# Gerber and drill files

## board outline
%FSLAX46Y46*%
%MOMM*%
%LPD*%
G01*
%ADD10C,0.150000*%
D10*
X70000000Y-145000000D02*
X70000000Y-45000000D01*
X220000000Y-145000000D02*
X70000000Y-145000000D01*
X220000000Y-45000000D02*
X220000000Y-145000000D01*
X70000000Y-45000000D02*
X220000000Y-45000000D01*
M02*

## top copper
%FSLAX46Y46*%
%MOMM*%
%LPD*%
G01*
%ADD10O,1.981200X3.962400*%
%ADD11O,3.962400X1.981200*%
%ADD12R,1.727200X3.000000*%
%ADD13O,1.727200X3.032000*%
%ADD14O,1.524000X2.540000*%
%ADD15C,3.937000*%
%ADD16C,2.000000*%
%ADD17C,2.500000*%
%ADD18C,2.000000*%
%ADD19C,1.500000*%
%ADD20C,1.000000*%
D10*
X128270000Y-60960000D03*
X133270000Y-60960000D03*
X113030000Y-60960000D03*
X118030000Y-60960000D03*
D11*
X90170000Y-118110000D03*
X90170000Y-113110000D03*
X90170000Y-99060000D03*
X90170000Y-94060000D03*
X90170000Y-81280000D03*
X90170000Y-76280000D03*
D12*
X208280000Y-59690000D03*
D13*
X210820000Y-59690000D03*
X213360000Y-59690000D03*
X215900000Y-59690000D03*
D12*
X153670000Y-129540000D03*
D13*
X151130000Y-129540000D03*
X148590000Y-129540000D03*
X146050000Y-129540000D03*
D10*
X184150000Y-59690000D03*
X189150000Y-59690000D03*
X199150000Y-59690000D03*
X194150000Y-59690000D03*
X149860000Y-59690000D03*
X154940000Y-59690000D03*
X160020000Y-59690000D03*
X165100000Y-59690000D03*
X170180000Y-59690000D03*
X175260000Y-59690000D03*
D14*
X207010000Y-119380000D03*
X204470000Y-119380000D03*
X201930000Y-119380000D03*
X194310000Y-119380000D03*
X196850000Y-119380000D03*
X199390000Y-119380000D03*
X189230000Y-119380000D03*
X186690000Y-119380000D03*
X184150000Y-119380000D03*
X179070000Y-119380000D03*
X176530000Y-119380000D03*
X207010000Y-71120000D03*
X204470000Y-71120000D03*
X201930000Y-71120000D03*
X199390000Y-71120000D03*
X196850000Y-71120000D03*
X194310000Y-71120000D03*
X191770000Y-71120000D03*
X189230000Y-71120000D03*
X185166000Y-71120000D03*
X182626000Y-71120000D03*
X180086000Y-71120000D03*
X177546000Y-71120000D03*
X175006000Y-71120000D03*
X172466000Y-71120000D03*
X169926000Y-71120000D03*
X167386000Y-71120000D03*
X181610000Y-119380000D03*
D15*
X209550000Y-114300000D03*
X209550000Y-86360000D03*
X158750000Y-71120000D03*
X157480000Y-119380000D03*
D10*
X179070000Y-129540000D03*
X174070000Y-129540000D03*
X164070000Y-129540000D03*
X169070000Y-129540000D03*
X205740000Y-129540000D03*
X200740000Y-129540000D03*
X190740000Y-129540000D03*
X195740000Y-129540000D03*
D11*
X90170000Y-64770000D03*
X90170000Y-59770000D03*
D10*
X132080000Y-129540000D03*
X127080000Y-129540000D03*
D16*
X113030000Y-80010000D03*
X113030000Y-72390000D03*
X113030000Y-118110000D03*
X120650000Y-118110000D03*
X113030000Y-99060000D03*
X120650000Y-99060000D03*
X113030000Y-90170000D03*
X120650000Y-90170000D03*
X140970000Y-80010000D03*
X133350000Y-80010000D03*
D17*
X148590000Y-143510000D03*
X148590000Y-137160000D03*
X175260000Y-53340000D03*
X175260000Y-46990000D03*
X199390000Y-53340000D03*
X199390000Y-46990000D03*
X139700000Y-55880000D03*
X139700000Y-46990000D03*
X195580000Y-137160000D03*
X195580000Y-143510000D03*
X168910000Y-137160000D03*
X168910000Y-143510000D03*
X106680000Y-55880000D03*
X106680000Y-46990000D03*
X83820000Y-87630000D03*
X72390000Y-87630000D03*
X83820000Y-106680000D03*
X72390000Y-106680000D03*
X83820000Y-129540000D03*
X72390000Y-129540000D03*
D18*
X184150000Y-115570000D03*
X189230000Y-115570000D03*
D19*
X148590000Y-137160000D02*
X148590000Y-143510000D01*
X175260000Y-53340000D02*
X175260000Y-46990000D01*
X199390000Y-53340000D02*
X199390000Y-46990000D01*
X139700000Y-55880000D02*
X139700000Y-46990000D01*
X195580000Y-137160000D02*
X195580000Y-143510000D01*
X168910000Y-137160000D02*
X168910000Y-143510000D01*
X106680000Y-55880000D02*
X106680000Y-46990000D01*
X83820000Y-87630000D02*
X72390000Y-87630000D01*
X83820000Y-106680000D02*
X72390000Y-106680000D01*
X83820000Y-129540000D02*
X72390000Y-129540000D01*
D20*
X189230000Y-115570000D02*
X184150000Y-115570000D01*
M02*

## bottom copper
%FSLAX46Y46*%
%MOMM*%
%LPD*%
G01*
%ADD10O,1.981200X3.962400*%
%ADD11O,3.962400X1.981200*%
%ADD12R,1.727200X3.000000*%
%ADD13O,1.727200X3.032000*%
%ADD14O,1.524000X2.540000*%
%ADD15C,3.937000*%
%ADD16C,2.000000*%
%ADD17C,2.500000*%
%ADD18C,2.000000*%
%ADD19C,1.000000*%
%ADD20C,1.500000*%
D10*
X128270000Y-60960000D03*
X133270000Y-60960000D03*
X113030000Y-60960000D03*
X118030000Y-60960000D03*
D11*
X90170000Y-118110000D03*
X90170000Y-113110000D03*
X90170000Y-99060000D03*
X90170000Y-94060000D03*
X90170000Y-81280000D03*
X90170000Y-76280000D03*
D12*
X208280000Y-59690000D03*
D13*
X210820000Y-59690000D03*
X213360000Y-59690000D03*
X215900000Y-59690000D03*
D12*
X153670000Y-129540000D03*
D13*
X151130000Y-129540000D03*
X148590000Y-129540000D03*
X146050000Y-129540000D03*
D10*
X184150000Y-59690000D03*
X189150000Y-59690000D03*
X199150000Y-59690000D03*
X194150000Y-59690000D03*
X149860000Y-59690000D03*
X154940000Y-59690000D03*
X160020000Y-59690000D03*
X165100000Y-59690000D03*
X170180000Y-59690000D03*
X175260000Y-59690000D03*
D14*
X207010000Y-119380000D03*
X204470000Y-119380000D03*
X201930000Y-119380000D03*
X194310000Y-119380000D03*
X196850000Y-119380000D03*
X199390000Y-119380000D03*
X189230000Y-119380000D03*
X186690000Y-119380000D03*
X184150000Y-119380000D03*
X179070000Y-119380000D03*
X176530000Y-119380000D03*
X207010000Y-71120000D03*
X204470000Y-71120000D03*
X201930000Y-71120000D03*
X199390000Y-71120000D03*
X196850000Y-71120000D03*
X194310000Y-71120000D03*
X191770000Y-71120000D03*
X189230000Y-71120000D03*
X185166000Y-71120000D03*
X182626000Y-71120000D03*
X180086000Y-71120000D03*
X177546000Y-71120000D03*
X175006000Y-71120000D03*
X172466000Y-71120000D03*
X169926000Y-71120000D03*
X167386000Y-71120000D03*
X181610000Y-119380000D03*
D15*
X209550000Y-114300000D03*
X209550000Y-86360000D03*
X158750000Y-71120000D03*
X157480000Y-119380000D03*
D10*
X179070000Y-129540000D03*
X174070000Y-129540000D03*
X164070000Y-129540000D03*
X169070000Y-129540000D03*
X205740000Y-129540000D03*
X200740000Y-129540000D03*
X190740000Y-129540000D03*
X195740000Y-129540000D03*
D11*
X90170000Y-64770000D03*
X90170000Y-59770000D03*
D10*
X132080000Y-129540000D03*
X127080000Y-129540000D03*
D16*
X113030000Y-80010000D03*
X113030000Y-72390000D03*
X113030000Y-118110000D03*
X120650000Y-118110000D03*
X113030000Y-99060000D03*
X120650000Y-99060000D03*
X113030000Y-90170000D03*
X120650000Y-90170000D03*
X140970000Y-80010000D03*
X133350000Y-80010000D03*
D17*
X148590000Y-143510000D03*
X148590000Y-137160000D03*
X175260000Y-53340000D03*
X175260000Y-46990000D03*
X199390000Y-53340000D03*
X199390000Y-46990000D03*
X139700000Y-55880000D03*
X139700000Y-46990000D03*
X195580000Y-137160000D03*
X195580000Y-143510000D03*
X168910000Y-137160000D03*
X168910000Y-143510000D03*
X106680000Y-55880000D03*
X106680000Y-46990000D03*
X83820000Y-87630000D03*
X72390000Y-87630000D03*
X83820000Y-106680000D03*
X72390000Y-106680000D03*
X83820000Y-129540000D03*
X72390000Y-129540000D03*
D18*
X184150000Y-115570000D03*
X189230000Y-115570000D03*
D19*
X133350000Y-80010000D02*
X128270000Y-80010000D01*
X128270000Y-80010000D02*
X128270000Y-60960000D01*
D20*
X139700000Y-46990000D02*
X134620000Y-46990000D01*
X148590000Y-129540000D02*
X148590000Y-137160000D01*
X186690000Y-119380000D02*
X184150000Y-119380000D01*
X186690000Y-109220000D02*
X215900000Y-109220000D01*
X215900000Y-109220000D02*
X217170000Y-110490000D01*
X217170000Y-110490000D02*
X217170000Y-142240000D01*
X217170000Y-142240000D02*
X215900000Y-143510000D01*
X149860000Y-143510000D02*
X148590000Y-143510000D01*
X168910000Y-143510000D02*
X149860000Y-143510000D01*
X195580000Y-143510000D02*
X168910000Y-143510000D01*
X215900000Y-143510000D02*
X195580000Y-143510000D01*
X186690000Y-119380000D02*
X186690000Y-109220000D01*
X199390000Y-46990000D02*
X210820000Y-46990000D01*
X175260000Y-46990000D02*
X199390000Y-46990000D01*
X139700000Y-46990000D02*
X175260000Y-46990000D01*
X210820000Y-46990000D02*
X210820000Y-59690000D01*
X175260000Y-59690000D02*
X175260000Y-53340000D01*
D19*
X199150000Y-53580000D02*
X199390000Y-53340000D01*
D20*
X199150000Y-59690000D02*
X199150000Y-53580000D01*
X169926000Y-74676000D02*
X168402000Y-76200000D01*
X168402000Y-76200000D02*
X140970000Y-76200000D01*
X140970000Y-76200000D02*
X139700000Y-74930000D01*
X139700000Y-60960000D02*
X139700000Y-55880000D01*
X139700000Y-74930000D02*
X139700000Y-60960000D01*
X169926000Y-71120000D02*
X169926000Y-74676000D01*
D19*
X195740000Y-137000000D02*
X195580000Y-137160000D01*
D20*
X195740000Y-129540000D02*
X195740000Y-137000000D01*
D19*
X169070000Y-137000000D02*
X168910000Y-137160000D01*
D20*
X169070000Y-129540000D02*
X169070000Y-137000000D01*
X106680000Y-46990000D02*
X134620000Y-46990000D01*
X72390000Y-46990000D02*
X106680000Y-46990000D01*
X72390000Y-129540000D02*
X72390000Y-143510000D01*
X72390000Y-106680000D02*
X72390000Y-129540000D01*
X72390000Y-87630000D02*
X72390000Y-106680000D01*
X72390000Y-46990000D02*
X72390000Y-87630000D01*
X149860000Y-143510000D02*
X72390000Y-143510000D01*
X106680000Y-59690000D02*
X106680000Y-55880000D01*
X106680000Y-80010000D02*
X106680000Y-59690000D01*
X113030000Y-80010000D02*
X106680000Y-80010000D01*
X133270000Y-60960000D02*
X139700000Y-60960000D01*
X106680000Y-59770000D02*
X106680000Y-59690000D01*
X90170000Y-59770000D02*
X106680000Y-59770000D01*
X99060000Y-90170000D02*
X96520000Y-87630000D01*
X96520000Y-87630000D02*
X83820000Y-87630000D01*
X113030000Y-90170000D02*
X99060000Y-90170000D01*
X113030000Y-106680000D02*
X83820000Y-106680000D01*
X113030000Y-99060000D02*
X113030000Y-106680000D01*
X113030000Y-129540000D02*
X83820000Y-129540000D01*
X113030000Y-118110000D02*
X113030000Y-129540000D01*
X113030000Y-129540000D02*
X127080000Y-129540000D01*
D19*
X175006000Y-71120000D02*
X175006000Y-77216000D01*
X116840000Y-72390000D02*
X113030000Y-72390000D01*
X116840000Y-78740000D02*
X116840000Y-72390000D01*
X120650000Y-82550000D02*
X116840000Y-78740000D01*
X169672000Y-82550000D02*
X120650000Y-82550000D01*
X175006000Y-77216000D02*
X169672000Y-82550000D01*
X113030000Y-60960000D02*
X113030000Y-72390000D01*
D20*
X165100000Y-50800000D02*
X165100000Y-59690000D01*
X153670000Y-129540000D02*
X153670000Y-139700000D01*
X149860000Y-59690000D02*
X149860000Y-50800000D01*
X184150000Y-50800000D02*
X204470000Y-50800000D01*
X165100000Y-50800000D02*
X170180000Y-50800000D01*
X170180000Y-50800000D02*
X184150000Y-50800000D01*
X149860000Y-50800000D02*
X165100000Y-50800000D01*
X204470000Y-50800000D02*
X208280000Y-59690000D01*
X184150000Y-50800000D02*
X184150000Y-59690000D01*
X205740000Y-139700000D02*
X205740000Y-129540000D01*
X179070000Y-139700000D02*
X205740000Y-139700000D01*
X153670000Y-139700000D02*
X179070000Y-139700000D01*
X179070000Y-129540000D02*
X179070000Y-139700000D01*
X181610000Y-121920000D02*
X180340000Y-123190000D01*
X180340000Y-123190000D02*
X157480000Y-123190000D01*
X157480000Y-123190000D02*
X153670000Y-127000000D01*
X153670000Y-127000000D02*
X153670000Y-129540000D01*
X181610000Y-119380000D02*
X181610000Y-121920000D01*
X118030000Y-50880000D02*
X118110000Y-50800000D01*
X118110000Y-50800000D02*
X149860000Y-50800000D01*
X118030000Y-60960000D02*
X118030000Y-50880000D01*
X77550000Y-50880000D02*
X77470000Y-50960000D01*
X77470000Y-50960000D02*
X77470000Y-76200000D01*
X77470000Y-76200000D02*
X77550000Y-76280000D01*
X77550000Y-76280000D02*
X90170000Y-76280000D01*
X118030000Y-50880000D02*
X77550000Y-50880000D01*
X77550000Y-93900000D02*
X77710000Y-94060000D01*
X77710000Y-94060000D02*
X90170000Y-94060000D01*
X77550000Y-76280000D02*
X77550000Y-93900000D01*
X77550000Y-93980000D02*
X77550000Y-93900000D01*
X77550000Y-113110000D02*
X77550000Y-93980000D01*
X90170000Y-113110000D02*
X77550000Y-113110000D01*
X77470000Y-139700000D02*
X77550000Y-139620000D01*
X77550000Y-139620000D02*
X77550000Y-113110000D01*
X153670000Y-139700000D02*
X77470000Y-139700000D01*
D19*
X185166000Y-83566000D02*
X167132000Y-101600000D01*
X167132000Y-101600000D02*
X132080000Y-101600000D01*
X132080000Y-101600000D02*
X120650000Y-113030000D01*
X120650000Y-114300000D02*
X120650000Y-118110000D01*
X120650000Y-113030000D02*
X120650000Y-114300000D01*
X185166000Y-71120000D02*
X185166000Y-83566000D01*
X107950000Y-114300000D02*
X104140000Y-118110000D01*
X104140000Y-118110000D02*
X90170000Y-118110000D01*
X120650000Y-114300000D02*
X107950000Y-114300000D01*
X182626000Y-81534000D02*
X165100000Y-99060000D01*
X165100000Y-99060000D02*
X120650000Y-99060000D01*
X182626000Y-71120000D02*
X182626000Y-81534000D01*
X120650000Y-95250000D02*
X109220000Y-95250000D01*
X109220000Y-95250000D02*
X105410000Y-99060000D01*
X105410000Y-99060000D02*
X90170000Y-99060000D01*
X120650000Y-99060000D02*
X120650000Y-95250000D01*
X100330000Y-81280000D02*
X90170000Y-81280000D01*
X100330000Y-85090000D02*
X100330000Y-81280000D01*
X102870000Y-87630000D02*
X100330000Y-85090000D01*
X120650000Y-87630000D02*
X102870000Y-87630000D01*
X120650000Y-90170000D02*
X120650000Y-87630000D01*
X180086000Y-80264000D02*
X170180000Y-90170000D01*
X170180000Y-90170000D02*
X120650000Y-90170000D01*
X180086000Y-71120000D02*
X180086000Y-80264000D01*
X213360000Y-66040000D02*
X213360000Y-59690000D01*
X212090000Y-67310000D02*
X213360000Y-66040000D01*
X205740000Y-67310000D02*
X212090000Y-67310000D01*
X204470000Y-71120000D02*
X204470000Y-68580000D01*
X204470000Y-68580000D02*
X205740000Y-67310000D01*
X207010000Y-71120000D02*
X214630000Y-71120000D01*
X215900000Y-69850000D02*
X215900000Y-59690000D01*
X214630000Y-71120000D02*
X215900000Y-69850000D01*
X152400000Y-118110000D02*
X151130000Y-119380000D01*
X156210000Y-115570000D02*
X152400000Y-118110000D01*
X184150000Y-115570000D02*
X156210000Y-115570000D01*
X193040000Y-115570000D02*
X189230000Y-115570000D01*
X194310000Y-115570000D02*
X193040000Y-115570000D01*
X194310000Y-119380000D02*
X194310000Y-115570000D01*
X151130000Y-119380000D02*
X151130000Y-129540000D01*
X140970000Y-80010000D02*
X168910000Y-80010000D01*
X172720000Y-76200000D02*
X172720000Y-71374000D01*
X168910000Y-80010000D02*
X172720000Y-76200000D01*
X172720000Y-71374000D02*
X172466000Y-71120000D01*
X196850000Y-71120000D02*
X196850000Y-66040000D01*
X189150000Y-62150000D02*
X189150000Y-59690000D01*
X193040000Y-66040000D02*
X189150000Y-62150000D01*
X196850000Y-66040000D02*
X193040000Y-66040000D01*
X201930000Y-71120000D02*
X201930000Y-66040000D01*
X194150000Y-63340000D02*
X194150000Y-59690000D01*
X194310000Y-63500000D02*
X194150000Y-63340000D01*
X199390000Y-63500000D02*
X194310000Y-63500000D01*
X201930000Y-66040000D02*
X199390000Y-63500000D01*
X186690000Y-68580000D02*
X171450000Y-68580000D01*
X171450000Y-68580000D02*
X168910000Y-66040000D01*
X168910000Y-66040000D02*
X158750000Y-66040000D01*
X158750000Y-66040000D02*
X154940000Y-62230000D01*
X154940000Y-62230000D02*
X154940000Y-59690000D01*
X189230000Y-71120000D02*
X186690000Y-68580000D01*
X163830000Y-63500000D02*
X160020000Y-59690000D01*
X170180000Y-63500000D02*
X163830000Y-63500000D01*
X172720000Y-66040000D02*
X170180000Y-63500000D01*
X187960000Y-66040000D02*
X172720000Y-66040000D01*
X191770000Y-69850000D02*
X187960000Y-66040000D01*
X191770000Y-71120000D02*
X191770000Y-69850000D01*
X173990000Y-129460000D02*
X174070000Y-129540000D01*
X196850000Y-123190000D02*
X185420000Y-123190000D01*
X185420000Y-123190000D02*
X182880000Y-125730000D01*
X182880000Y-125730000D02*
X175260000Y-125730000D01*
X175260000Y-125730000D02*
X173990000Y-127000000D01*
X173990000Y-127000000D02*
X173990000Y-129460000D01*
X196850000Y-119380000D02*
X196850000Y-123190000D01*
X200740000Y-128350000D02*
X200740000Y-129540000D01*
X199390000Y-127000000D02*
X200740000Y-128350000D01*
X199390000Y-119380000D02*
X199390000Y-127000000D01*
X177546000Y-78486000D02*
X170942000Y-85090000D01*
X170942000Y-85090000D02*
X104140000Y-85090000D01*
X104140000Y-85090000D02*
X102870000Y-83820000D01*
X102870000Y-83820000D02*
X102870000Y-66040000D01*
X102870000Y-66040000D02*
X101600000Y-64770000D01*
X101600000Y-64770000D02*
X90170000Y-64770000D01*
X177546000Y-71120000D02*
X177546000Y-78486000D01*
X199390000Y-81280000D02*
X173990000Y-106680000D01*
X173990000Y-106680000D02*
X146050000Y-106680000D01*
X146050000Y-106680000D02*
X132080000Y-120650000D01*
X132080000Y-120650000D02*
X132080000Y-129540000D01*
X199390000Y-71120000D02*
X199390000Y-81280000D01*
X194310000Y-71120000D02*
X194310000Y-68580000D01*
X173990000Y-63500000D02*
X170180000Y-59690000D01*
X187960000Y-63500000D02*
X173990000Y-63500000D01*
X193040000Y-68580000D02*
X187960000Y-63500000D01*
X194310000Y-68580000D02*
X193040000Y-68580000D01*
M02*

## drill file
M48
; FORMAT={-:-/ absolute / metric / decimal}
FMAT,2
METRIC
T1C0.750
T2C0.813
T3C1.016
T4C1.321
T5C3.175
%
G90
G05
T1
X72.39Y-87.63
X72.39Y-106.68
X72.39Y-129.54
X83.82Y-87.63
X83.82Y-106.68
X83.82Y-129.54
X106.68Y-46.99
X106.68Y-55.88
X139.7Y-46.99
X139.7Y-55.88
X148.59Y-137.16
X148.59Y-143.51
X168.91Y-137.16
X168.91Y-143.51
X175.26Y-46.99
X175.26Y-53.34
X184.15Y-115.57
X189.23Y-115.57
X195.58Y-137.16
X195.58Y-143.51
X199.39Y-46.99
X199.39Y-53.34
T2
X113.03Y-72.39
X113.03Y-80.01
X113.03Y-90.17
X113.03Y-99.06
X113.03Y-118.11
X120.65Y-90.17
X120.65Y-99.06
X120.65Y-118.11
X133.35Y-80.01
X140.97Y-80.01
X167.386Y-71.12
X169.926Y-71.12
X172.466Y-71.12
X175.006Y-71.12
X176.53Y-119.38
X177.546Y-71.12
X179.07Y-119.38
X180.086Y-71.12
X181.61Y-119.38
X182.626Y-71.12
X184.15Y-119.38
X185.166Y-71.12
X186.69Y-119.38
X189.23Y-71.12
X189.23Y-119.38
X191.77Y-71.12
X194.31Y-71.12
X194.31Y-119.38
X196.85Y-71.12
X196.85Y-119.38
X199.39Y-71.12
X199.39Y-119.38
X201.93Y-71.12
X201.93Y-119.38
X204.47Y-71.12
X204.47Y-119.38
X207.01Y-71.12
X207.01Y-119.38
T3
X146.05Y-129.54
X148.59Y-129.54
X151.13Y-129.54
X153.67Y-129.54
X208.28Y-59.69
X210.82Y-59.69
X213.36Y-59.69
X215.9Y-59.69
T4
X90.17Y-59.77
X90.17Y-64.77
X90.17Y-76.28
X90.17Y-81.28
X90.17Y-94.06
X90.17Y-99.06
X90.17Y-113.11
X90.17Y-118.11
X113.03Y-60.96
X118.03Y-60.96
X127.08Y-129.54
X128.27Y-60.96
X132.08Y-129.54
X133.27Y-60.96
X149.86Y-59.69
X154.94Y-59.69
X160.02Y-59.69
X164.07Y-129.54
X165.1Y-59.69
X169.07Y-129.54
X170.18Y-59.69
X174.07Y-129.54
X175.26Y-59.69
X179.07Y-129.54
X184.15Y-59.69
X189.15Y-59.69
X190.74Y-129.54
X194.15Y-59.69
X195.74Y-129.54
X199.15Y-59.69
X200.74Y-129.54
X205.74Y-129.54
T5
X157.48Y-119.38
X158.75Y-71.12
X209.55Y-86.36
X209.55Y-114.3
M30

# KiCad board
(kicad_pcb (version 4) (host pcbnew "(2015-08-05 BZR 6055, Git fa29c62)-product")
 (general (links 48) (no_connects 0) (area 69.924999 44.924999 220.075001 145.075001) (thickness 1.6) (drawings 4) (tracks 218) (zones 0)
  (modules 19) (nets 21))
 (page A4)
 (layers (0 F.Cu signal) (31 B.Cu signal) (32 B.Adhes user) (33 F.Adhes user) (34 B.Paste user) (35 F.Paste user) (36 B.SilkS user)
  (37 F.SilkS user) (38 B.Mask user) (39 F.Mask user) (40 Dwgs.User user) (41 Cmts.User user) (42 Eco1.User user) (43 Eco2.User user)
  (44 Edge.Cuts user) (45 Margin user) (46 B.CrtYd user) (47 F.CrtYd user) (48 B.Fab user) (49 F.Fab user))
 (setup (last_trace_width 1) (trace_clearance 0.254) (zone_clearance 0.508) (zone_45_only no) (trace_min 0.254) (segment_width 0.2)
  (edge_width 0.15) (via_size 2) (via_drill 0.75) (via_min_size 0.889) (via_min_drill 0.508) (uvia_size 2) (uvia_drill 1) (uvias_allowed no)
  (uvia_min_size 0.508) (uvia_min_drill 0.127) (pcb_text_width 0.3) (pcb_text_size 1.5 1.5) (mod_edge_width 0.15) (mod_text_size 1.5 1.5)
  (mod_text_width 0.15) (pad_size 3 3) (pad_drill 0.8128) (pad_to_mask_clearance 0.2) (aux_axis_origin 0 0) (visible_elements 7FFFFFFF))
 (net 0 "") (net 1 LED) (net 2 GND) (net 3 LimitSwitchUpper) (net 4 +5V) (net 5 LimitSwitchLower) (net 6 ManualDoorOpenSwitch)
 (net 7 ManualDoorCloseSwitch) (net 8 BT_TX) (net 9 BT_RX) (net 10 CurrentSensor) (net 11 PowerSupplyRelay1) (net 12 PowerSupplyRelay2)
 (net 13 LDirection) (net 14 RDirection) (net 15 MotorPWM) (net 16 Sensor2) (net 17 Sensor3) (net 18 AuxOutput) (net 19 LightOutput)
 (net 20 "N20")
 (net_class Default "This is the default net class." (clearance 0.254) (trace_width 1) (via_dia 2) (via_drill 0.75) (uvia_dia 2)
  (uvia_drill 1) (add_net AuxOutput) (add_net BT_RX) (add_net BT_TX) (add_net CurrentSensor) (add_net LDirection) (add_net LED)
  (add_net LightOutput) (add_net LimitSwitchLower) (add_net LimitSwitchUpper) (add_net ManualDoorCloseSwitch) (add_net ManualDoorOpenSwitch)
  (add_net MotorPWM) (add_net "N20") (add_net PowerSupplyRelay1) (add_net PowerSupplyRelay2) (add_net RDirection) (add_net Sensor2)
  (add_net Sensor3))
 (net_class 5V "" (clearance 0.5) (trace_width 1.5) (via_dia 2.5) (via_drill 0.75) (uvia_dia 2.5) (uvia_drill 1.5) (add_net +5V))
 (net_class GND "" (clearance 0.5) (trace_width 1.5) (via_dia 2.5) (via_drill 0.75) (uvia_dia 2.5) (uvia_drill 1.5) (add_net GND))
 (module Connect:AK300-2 (layer F.Cu) (at 128.27 60.96)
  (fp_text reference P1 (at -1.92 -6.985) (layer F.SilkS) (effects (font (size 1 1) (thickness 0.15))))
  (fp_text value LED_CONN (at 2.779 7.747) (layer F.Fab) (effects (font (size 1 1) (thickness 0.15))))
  (pad 1 thru_hole oval (at 0 0) (size 1.9812 3.9624) (drill 1.3208) (layers *.Cu F.Paste F.SilkS F.Mask) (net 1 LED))
  (pad 2 thru_hole oval (at 5 0) (size 1.9812 3.9624) (drill 1.3208) (layers *.Cu F.Paste F.SilkS F.Mask) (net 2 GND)))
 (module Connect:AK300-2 (layer F.Cu) (at 113.03 60.96)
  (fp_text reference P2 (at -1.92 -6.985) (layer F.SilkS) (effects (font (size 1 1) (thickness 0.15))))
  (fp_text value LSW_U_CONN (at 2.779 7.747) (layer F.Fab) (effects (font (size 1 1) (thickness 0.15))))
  (pad 1 thru_hole oval (at 0 0) (size 1.9812 3.9624) (drill 1.3208) (layers *.Cu F.Paste F.SilkS F.Mask) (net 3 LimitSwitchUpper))
  (pad 2 thru_hole oval (at 5 0) (size 1.9812 3.9624) (drill 1.3208) (layers *.Cu F.Paste F.SilkS F.Mask) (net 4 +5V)))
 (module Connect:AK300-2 (layer F.Cu) (at 90.17 118.11 90)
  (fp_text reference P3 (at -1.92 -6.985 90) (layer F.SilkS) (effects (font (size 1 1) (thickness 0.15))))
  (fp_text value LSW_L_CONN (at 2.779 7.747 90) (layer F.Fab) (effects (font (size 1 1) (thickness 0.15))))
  (pad 1 thru_hole oval (at 0 0 90) (size 1.9812 3.9624) (drill 1.3208) (layers *.Cu F.Paste F.SilkS F.Mask) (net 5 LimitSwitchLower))
  (pad 2 thru_hole oval (at 5 0 90) (size 1.9812 3.9624) (drill 1.3208) (layers *.Cu F.Paste F.SilkS F.Mask) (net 4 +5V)))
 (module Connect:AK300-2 (layer F.Cu) (at 90.17 99.06 90)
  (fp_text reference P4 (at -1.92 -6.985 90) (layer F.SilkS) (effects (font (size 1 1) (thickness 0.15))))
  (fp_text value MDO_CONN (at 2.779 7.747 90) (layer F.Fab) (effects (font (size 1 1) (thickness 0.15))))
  (pad 1 thru_hole oval (at 0 0 90) (size 1.9812 3.9624) (drill 1.3208) (layers *.Cu F.Paste F.SilkS F.Mask) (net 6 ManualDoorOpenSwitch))
  (pad 2 thru_hole oval (at 5 0 90) (size 1.9812 3.9624) (drill 1.3208) (layers *.Cu F.Paste F.SilkS F.Mask) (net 4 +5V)))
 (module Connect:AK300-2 (layer F.Cu) (at 90.17 81.28 90)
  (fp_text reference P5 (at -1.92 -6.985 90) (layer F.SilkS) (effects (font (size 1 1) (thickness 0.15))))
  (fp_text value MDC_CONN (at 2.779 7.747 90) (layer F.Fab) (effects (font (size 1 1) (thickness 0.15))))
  (pad 1 thru_hole oval (at 0 0 90) (size 1.9812 3.9624) (drill 1.3208) (layers *.Cu F.Paste F.SilkS F.Mask) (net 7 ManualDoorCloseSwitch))
  (pad 2 thru_hole oval (at 5 0 90) (size 1.9812 3.9624) (drill 1.3208) (layers *.Cu F.Paste F.SilkS F.Mask) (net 4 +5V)))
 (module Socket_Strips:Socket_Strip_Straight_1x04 (layer F.Cu) (at 208.28 59.69)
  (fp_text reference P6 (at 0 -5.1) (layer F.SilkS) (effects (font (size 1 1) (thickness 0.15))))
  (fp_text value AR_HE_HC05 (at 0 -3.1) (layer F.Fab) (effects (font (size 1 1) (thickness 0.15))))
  (pad 1 thru_hole rect (at 0 0) (size 1.7272 3) (drill 1.016) (layers *.Cu *.Mask F.SilkS) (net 4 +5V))
  (pad 2 thru_hole oval (at 2.54 0) (size 1.7272 3.032) (drill 1.016) (layers *.Cu *.Mask F.SilkS) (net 2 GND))
  (pad 3 thru_hole oval (at 5.08 0) (size 1.7272 3.032) (drill 1.016) (layers *.Cu *.Mask F.SilkS) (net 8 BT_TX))
  (pad 4 thru_hole oval (at 7.62 0) (size 1.7272 3.032) (drill 1.016) (layers *.Cu *.Mask F.SilkS) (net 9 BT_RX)))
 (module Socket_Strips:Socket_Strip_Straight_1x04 (layer F.Cu) (at 153.67 129.54 180)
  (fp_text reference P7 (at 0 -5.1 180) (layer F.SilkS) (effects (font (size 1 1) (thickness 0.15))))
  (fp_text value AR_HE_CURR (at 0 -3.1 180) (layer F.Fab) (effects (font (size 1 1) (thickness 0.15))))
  (pad 1 thru_hole rect (at 0 0 180) (size 1.7272 3) (drill 1.016) (layers *.Cu *.Mask F.SilkS) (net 4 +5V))
  (pad 2 thru_hole oval (at 2.54 0 180) (size 1.7272 3.032) (drill 1.016) (layers *.Cu *.Mask F.SilkS) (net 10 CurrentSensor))
  (pad 3 thru_hole oval (at 5.08 0 180) (size 1.7272 3.032) (drill 1.016) (layers *.Cu *.Mask F.SilkS) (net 2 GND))
  (pad 4 thru_hole oval (at 7.62 0 180) (size 1.7272 3.032) (drill 1.016) (layers *.Cu *.Mask F.SilkS)))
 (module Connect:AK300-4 (layer F.Cu) (at 184.15 59.69)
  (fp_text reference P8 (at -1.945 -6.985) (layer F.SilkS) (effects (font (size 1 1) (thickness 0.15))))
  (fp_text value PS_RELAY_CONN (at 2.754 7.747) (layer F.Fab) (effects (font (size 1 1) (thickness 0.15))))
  (pad 1 thru_hole oval (at 0 0) (size 1.9812 3.9624) (drill 1.3208) (layers *.Cu F.Paste F.SilkS F.Mask) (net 4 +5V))
  (pad 2 thru_hole oval (at 5 0) (size 1.9812 3.9624) (drill 1.3208) (layers *.Cu F.Paste F.SilkS F.Mask) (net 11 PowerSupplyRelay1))
  (pad 4 thru_hole oval (at 15 0) (size 1.9812 3.9624) (drill 1.3208) (layers *.Cu F.Paste F.SilkS F.Mask) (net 2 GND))
  (pad 3 thru_hole oval (at 10 0) (size 1.9812 3.9624) (drill 1.3208) (layers *.Cu *.Mask F.SilkS) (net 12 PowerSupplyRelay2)))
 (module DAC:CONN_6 (layer F.Cu) (at 162.56 59.69)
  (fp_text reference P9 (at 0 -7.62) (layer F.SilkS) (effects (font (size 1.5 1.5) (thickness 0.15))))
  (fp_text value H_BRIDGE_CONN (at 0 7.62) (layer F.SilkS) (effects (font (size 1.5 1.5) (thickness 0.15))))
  (pad 1 thru_hole oval (at -12.7 0) (size 1.9812 3.9624) (drill 1.3208) (layers *.Cu *.Mask F.SilkS) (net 4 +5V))
  (pad 2 thru_hole oval (at -7.62 0) (size 1.9812 3.9624) (drill 1.3208) (layers *.Cu *.Mask F.SilkS) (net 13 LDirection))
  (pad 3 thru_hole oval (at -2.54 0) (size 1.9812 3.9624) (drill 1.3208) (layers *.Cu *.Mask F.SilkS) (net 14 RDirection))
  (pad 4 thru_hole oval (at 2.54 0) (size 1.9812 3.9624) (drill 1.3208) (layers *.Cu *.Mask F.SilkS) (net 4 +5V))
  (pad 5 thru_hole oval (at 7.62 0) (size 1.9812 3.9624) (drill 1.3208) (layers *.Cu *.Mask F.SilkS) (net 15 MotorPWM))
  (pad 6 thru_hole oval (at 12.7 0) (size 1.9812 3.9624) (drill 1.3208) (layers *.Cu *.Mask F.SilkS) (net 2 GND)))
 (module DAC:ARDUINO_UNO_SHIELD (layer F.Cu) (at 143.51 121.92)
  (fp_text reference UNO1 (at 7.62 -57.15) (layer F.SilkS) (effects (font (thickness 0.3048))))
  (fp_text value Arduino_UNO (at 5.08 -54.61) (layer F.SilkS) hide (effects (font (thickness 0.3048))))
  (pad AD5 thru_hole oval (at 63.5 -2.54 90) (size 2.54 1.524) (drill 0.8128) (layers *.Cu *.Mask F.SilkS))
  (pad AD4 thru_hole oval (at 60.96 -2.54 90) (size 2.54 1.524) (drill 0.8128) (layers *.Cu *.Mask F.SilkS))
  (pad AD3 thru_hole oval (at 58.42 -2.54 90) (size 2.54 1.524) (drill 0.8128) (layers *.Cu *.Mask F.SilkS))
  (pad AD0 thru_hole oval (at 50.8 -2.54 90) (size 2.54 1.524) (drill 0.8128) (layers *.Cu *.Mask F.SilkS) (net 10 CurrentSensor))
  (pad AD1 thru_hole oval (at 53.34 -2.54 90) (size 2.54 1.524) (drill 0.8128) (layers *.Cu *.Mask F.SilkS) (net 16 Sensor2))
  (pad AD2 thru_hole oval (at 55.88 -2.54 90) (size 2.54 1.524) (drill 0.8128) (layers *.Cu *.Mask F.SilkS) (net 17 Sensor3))
  (pad V_IN thru_hole oval (at 45.72 -2.54 90) (size 2.54 1.524) (drill 0.8128) (layers *.Cu *.Mask F.SilkS))
  (pad GND2 thru_hole oval (at 43.18 -2.54 90) (size 2.54 1.524) (drill 0.8128) (layers *.Cu *.Mask F.SilkS) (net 2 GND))
  (pad GND1 thru_hole oval (at 40.64 -2.54 90) (size 2.54 1.524) (drill 0.8128) (layers *.Cu *.Mask F.SilkS) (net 2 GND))
  (pad 3V3 thru_hole oval (at 35.56 -2.54 90) (size 2.54 1.524) (drill 0.8128) (layers *.Cu *.Mask F.SilkS))
  (pad RST thru_hole oval (at 33.02 -2.54 90) (size 2.54 1.524) (drill 0.8128) (layers *.Cu *.Mask F.SilkS))
  (pad 0 thru_hole oval (at 63.5 -50.8 90) (size 2.54 1.524) (drill 0.8128) (layers *.Cu *.Mask F.SilkS) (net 9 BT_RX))
  (pad 1 thru_hole oval (at 60.96 -50.8 90) (size 2.54 1.524) (drill 0.8128) (layers *.Cu *.Mask F.SilkS) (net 8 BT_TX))
  (pad 2 thru_hole oval (at 58.42 -50.8 90) (size 2.54 1.524) (drill 0.8128) (layers *.Cu *.Mask F.SilkS) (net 12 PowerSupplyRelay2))
  (pad 3 thru_hole oval (at 55.88 -50.8 90) (size 2.54 1.524) (drill 0.8128) (layers *.Cu *.Mask F.SilkS) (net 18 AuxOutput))
  (pad 4 thru_hole oval (at 53.34 -50.8 90) (size 2.54 1.524) (drill 0.8128) (layers *.Cu *.Mask F.SilkS) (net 11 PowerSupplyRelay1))
  (pad 5 thru_hole oval (at 50.8 -50.8 90) (size 2.54 1.524) (drill 0.8128) (layers *.Cu *.Mask F.SilkS) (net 15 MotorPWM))
  (pad 6 thru_hole oval (at 48.26 -50.8 90) (size 2.54 1.524) (drill 0.8128) (layers *.Cu *.Mask F.SilkS) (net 14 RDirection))
  (pad 7 thru_hole oval (at 45.72 -50.8 90) (size 2.54 1.524) (drill 0.8128) (layers *.Cu *.Mask F.SilkS) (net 13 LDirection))
  (pad 8 thru_hole oval (at 41.656 -50.8 90) (size 2.54 1.524) (drill 0.8128) (layers *.Cu *.Mask F.SilkS) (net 5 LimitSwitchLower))
  (pad 9 thru_hole oval (at 39.116 -50.8 90) (size 2.54 1.524) (drill 0.8128) (layers *.Cu *.Mask F.SilkS) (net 6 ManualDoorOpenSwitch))
  (pad 10 thru_hole oval (at 36.576 -50.8 90) (size 2.54 1.524) (drill 0.8128) (layers *.Cu *.Mask F.SilkS) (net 7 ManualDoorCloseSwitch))
  (pad 11 thru_hole oval (at 34.036 -50.8 90) (size 2.54 1.524) (drill 0.8128) (layers *.Cu *.Mask F.SilkS) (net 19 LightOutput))
  (pad 12 thru_hole oval (at 31.496 -50.8 90) (size 2.54 1.524) (drill 0.8128) (layers *.Cu *.Mask F.SilkS) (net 3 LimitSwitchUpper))
  (pad 13 thru_hole oval (at 28.956 -50.8 90) (size 2.54 1.524) (drill 0.8128) (layers *.Cu *.Mask F.SilkS) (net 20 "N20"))
  (pad GND3 thru_hole oval (at 26.416 -50.8 90) (size 2.54 1.524) (drill 0.8128) (layers *.Cu *.Mask F.SilkS) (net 2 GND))
  (pad AREF thru_hole oval (at 23.876 -50.8 90) (size 2.54 1.524) (drill 0.8128) (layers *.Cu *.Mask F.SilkS))
  (pad 5V thru_hole oval (at 38.1 -2.54 90) (size 2.54 1.524) (drill 0.8128) (layers *.Cu *.Mask F.SilkS) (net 4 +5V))
  (pad "" thru_hole circle (at 66.04 -7.62 90) (size 3.937 3.937) (drill 3.175) (layers *.Cu *.Mask F.SilkS))
  (pad "" thru_hole circle (at 66.04 -35.56 90) (size 3.937 3.937) (drill 3.175) (layers *.Cu *.Mask F.SilkS))
  (pad "" thru_hole circle (at 15.24 -50.8 90) (size 3.937 3.937) (drill 3.175) (layers *.Cu *.Mask F.SilkS))
  (pad "" thru_hole circle (at 13.97 -2.54 90) (size 3.937 3.937) (drill 3.175) (layers *.Cu *.Mask F.SilkS)))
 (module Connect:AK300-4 (layer F.Cu) (at 179.07 129.54 180)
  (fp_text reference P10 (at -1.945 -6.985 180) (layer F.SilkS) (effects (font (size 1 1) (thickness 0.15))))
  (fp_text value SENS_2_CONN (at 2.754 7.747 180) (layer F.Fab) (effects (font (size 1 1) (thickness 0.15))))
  (pad 1 thru_hole oval (at 0 0 180) (size 1.9812 3.9624) (drill 1.3208) (layers *.Cu F.Paste F.SilkS F.Mask) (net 4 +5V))
  (pad 2 thru_hole oval (at 5 0 180) (size 1.9812 3.9624) (drill 1.3208) (layers *.Cu F.Paste F.SilkS F.Mask) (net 16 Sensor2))
  (pad 4 thru_hole oval (at 15 0 180) (size 1.9812 3.9624) (drill 1.3208) (layers *.Cu F.Paste F.SilkS F.Mask))
  (pad 3 thru_hole oval (at 10 0 180) (size 1.9812 3.9624) (drill 1.3208) (layers *.Cu *.Mask F.SilkS) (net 2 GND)))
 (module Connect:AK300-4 (layer F.Cu) (at 205.74 129.54 180)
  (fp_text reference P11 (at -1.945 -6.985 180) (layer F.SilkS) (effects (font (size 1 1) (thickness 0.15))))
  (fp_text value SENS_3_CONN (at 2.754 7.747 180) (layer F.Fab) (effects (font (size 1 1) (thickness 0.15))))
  (pad 1 thru_hole oval (at 0 0 180) (size 1.9812 3.9624) (drill 1.3208) (layers *.Cu F.Paste F.SilkS F.Mask) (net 4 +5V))
  (pad 2 thru_hole oval (at 5 0 180) (size 1.9812 3.9624) (drill 1.3208) (layers *.Cu F.Paste F.SilkS F.Mask) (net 17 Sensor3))
  (pad 4 thru_hole oval (at 15 0 180) (size 1.9812 3.9624) (drill 1.3208) (layers *.Cu F.Paste F.SilkS F.Mask))
  (pad 3 thru_hole oval (at 10 0 180) (size 1.9812 3.9624) (drill 1.3208) (layers *.Cu *.Mask F.SilkS) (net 2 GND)))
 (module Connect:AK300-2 (layer F.Cu) (at 90.17 64.77 90)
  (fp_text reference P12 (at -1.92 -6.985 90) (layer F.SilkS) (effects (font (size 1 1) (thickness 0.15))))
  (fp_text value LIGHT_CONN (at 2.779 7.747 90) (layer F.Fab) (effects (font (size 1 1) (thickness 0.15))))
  (pad 1 thru_hole oval (at 0 0 90) (size 1.9812 3.9624) (drill 1.3208) (layers *.Cu F.Paste F.SilkS F.Mask) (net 19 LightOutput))
  (pad 2 thru_hole oval (at 5 0 90) (size 1.9812 3.9624) (drill 1.3208) (layers *.Cu F.Paste F.SilkS F.Mask) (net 2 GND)))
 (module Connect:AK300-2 (layer F.Cu) (at 132.08 129.54 180)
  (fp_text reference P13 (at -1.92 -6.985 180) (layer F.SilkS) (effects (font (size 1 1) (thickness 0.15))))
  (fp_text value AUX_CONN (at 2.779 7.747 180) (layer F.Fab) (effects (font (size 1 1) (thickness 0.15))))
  (pad 1 thru_hole oval (at 0 0 180) (size 1.9812 3.9624) (drill 1.3208) (layers *.Cu F.Paste F.SilkS F.Mask) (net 18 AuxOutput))
  (pad 2 thru_hole oval (at 5 0 180) (size 1.9812 3.9624) (drill 1.3208) (layers *.Cu F.Paste F.SilkS F.Mask) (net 2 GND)))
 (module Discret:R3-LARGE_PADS (layer F.Cu) (at 113.03 76.2 90)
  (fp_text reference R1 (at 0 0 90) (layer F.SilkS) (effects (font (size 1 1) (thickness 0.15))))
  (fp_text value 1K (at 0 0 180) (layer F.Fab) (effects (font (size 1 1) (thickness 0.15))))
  (pad 1 thru_hole circle (at -3.81 0 90) (size 2 2) (drill 0.8128) (layers *.Cu *.Mask F.SilkS) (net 2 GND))
  (pad 2 thru_hole circle (at 3.81 0 90) (size 2 2) (drill 0.8128) (layers *.Cu *.Mask F.SilkS) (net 3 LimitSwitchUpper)))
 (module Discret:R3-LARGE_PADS (layer F.Cu) (at 116.84 118.11)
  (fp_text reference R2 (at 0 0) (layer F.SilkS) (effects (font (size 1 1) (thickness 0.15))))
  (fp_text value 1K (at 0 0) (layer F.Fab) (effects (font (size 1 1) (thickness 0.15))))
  (pad 1 thru_hole circle (at -3.81 0) (size 2 2) (drill 0.8128) (layers *.Cu *.Mask F.SilkS) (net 2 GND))
  (pad 2 thru_hole circle (at 3.81 0) (size 2 2) (drill 0.8128) (layers *.Cu *.Mask F.SilkS) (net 5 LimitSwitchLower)))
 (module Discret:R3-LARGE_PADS (layer F.Cu) (at 116.84 99.06)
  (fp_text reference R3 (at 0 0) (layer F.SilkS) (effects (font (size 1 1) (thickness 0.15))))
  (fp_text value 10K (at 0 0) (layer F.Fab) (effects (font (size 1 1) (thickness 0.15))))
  (pad 1 thru_hole circle (at -3.81 0) (size 2 2) (drill 0.8128) (layers *.Cu *.Mask F.SilkS) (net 2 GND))
  (pad 2 thru_hole circle (at 3.81 0) (size 2 2) (drill 0.8128) (layers *.Cu *.Mask F.SilkS) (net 6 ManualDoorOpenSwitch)))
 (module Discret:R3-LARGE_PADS (layer F.Cu) (at 116.84 90.17)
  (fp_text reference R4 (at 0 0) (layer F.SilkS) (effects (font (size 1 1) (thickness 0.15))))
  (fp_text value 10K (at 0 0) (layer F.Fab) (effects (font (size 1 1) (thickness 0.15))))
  (pad 1 thru_hole circle (at -3.81 0) (size 2 2) (drill 0.8128) (layers *.Cu *.Mask F.SilkS) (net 2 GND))
  (pad 2 thru_hole circle (at 3.81 0) (size 2 2) (drill 0.8128) (layers *.Cu *.Mask F.SilkS) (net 7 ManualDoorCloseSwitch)))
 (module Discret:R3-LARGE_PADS (layer F.Cu) (at 137.16 80.01 180)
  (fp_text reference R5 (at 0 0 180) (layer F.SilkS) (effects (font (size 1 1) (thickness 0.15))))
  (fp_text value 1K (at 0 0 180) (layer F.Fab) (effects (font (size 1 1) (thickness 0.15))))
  (pad 1 thru_hole circle (at -3.81 0 180) (size 2 2) (drill 0.8128) (layers *.Cu *.Mask F.SilkS) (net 20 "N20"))
  (pad 2 thru_hole circle (at 3.81 0 180) (size 2 2) (drill 0.8128) (layers *.Cu *.Mask F.SilkS) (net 1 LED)))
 (gr_line (start 70 145) (end 70 45) (angle 90) (layer Edge.Cuts) (width 0.15))
 (gr_line (start 220 145) (end 70 145) (angle 90) (layer Edge.Cuts) (width 0.15))
 (gr_line (start 220 45) (end 220 145) (angle 90) (layer Edge.Cuts) (width 0.15))
 (gr_line (start 70 45) (end 220 45) (angle 90) (layer Edge.Cuts) (width 0.15))
 (segment (start 133.35 80.01) (end 128.27 80.01) (width 1) (layer B.Cu) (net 1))
 (segment (start 128.27 80.01) (end 128.27 60.96) (width 1) (layer B.Cu) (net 1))
 (segment (start 139.7 46.99) (end 134.62 46.99) (width 1.5) (layer B.Cu) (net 2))
 (segment (start 148.59 129.54) (end 148.59 137.16) (width 1.5) (layer B.Cu) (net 2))
 (via (at 148.59 143.51) (size 2.5) (layers F.Cu B.Cu) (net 2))
 (segment (start 148.59 137.16) (end 148.59 143.51) (width 1.5) (layer F.Cu) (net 2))
 (via (at 148.59 137.16) (size 2.5) (layers F.Cu B.Cu) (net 2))
 (segment (start 186.69 119.38) (end 184.15 119.38) (width 1.5) (layer B.Cu) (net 2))
 (segment (start 186.69 109.22) (end 215.9 109.22) (width 1.5) (layer B.Cu) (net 2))
 (segment (start 215.9 109.22) (end 217.17 110.49) (width 1.5) (layer B.Cu) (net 2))
 (segment (start 217.17 110.49) (end 217.17 142.24) (width 1.5) (layer B.Cu) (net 2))
 (segment (start 217.17 142.24) (end 215.9 143.51) (width 1.5) (layer B.Cu) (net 2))
 (segment (start 149.86 143.51) (end 148.59 143.51) (width 1.5) (layer B.Cu) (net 2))
 (segment (start 168.91 143.51) (end 149.86 143.51) (width 1.5) (layer B.Cu) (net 2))
 (segment (start 195.58 143.51) (end 168.91 143.51) (width 1.5) (layer B.Cu) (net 2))
 (segment (start 215.9 143.51) (end 195.58 143.51) (width 1.5) (layer B.Cu) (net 2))
 (segment (start 186.69 119.38) (end 186.69 109.22) (width 1.5) (layer B.Cu) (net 2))
 (segment (start 199.39 46.99) (end 210.82 46.99) (width 1.5) (layer B.Cu) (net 2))
 (segment (start 175.26 46.99) (end 199.39 46.99) (width 1.5) (layer B.Cu) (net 2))
 (segment (start 139.7 46.99) (end 175.26 46.99) (width 1.5) (layer B.Cu) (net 2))
 (segment (start 210.82 46.99) (end 210.82 59.69) (width 1.5) (layer B.Cu) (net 2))
 (via (at 175.26 53.34) (size 2.5) (layers F.Cu B.Cu) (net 2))
 (segment (start 175.26 53.34) (end 175.26 46.99) (width 1.5) (layer F.Cu) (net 2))
 (via (at 175.26 46.99) (size 2.5) (layers F.Cu B.Cu) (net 2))
 (segment (start 175.26 59.69) (end 175.26 53.34) (width 1.5) (layer B.Cu) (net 2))
 (segment (start 199.15 53.58) (end 199.39 53.34) (width 1) (layer B.Cu) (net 2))
 (via (at 199.39 53.34) (size 2.5) (layers F.Cu B.Cu) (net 2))
 (segment (start 199.39 53.34) (end 199.39 46.99) (width 1.5) (layer F.Cu) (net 2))
 (via (at 199.39 46.99) (size 2.5) (layers F.Cu B.Cu) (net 2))
 (segment (start 199.15 59.69) (end 199.15 53.58) (width 1.5) (layer B.Cu) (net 2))
 (segment (start 169.926 74.676) (end 168.402 76.2) (width 1.5) (layer B.Cu) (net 2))
 (segment (start 168.402 76.2) (end 140.97 76.2) (width 1.5) (layer B.Cu) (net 2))
 (segment (start 140.97 76.2) (end 139.7 74.93) (width 1.5) (layer B.Cu) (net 2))
 (segment (start 139.7 60.96) (end 139.7 55.88) (width 1.5) (layer B.Cu) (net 2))
 (segment (start 139.7 74.93) (end 139.7 60.96) (width 1.5) (layer B.Cu) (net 2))
 (via (at 139.7 55.88) (size 2.5) (layers F.Cu B.Cu) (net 2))
 (segment (start 139.7 55.88) (end 139.7 46.99) (width 1.5) (layer F.Cu) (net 2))
 (via (at 139.7 46.99) (size 2.5) (layers F.Cu B.Cu) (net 2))
 (segment (start 169.926 71.12) (end 169.926 74.676) (width 1.5) (layer B.Cu) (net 2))
 (segment (start 195.74 137) (end 195.58 137.16) (width 1) (layer B.Cu) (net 2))
 (via (at 195.58 137.16) (size 2.5) (layers F.Cu B.Cu) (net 2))
 (segment (start 195.58 137.16) (end 195.58 143.51) (width 1.5) (layer F.Cu) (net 2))
 (via (at 195.58 143.51) (size 2.5) (layers F.Cu B.Cu) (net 2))
 (segment (start 195.74 129.54) (end 195.74 137) (width 1.5) (layer B.Cu) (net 2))
 (segment (start 169.07 137) (end 168.91 137.16) (width 1) (layer B.Cu) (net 2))
 (via (at 168.91 137.16) (size 2.5) (layers F.Cu B.Cu) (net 2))
 (segment (start 168.91 137.16) (end 168.91 143.51) (width 1.5) (layer F.Cu) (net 2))
 (via (at 168.91 143.51) (size 2.5) (layers F.Cu B.Cu) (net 2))
 (segment (start 169.07 129.54) (end 169.07 137) (width 1.5) (layer B.Cu) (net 2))
 (segment (start 106.68 46.99) (end 134.62 46.99) (width 1.5) (layer B.Cu) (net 2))
 (segment (start 72.39 46.99) (end 106.68 46.99) (width 1.5) (layer B.Cu) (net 2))
 (segment (start 72.39 129.54) (end 72.39 143.51) (width 1.5) (layer B.Cu) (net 2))
 (segment (start 72.39 106.68) (end 72.39 129.54) (width 1.5) (layer B.Cu) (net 2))
 (segment (start 72.39 87.63) (end 72.39 106.68) (width 1.5) (layer B.Cu) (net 2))
 (segment (start 72.39 46.99) (end 72.39 87.63) (width 1.5) (layer B.Cu) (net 2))
 (segment (start 149.86 143.51) (end 72.39 143.51) (width 1.5) (layer B.Cu) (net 2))
 (segment (start 106.68 59.69) (end 106.68 55.88) (width 1.5) (layer B.Cu) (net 2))
 (segment (start 106.68 80.01) (end 106.68 59.69) (width 1.5) (layer B.Cu) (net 2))
 (via (at 106.68 55.88) (size 2.5) (layers F.Cu B.Cu) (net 2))
 (segment (start 106.68 55.88) (end 106.68 46.99) (width 1.5) (layer F.Cu) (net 2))
 (via (at 106.68 46.99) (size 2.5) (layers F.Cu B.Cu) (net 2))
 (segment (start 113.03 80.01) (end 106.68 80.01) (width 1.5) (layer B.Cu) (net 2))
 (segment (start 133.27 60.96) (end 139.7 60.96) (width 1.5) (layer B.Cu) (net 2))
 (segment (start 106.68 59.77) (end 106.68 59.69) (width 1.5) (layer B.Cu) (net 2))
 (segment (start 90.17 59.77) (end 106.68 59.77) (width 1.5) (layer B.Cu) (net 2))
 (segment (start 99.06 90.17) (end 96.52 87.63) (width 1.5) (layer B.Cu) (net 2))
 (segment (start 96.52 87.63) (end 83.82 87.63) (width 1.5) (layer B.Cu) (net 2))
 (via (at 83.82 87.63) (size 2.5) (layers F.Cu B.Cu) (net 2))
 (segment (start 83.82 87.63) (end 72.39 87.63) (width 1.5) (layer F.Cu) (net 2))
 (via (at 72.39 87.63) (size 2.5) (layers F.Cu B.Cu) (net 2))
 (segment (start 113.03 90.17) (end 99.06 90.17) (width 1.5) (layer B.Cu) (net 2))
 (segment (start 113.03 106.68) (end 83.82 106.68) (width 1.5) (layer B.Cu) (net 2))
 (via (at 83.82 106.68) (size 2.5) (layers F.Cu B.Cu) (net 2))
 (segment (start 83.82 106.68) (end 72.39 106.68) (width 1.5) (layer F.Cu) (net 2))
 (via (at 72.39 106.68) (size 2.5) (layers F.Cu B.Cu) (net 2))
 (segment (start 113.03 99.06) (end 113.03 106.68) (width 1.5) (layer B.Cu) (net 2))
 (segment (start 113.03 129.54) (end 83.82 129.54) (width 1.5) (layer B.Cu) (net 2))
 (via (at 83.82 129.54) (size 2.5) (layers F.Cu B.Cu) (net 2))
 (segment (start 83.82 129.54) (end 72.39 129.54) (width 1.5) (layer F.Cu) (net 2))
 (via (at 72.39 129.54) (size 2.5) (layers F.Cu B.Cu) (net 2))
 (segment (start 113.03 118.11) (end 113.03 129.54) (width 1.5) (layer B.Cu) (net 2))
 (segment (start 113.03 129.54) (end 127.08 129.54) (width 1.5) (layer B.Cu) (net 2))
 (segment (start 175.006 71.12) (end 175.006 77.216) (width 1) (layer B.Cu) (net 3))
 (segment (start 116.84 72.39) (end 113.03 72.39) (width 1) (layer B.Cu) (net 3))
 (segment (start 116.84 78.74) (end 116.84 72.39) (width 1) (layer B.Cu) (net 3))
 (segment (start 120.65 82.55) (end 116.84 78.74) (width 1) (layer B.Cu) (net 3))
 (segment (start 169.672 82.55) (end 120.65 82.55) (width 1) (layer B.Cu) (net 3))
 (segment (start 175.006 77.216) (end 169.672 82.55) (width 1) (layer B.Cu) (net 3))
 (segment (start 113.03 60.96) (end 113.03 72.39) (width 1) (layer B.Cu) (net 3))
 (segment (start 165.1 50.8) (end 165.1 59.69) (width 1.5) (layer B.Cu) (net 4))
 (segment (start 153.67 129.54) (end 153.67 139.7) (width 1.5) (layer B.Cu) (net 4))
 (segment (start 149.86 59.69) (end 149.86 50.8) (width 1.5) (layer B.Cu) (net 4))
 (segment (start 184.15 50.8) (end 204.47 50.8) (width 1.5) (layer B.Cu) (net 4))
 (segment (start 165.1 50.8) (end 170.18 50.8) (width 1.5) (layer B.Cu) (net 4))
 (segment (start 170.18 50.8) (end 184.15 50.8) (width 1.5) (layer B.Cu) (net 4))
 (segment (start 149.86 50.8) (end 165.1 50.8) (width 1.5) (layer B.Cu) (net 4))
 (segment (start 204.47 50.8) (end 208.28 59.69) (width 1.5) (layer B.Cu) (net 4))
 (segment (start 184.15 50.8) (end 184.15 59.69) (width 1.5) (layer B.Cu) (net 4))
 (segment (start 205.74 139.7) (end 205.74 129.54) (width 1.5) (layer B.Cu) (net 4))
 (segment (start 179.07 139.7) (end 205.74 139.7) (width 1.5) (layer B.Cu) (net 4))
 (segment (start 153.67 139.7) (end 179.07 139.7) (width 1.5) (layer B.Cu) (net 4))
 (segment (start 179.07 129.54) (end 179.07 139.7) (width 1.5) (layer B.Cu) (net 4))
 (segment (start 181.61 121.92) (end 180.34 123.19) (width 1.5) (layer B.Cu) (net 4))
 (segment (start 180.34 123.19) (end 157.48 123.19) (width 1.5) (layer B.Cu) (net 4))
 (segment (start 157.48 123.19) (end 153.67 127) (width 1.5) (layer B.Cu) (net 4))
 (segment (start 153.67 127) (end 153.67 129.54) (width 1.5) (layer B.Cu) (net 4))
 (segment (start 181.61 119.38) (end 181.61 121.92) (width 1.5) (layer B.Cu) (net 4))
 (segment (start 118.03 50.88) (end 118.11 50.8) (width 1.5) (layer B.Cu) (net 4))
 (segment (start 118.11 50.8) (end 149.86 50.8) (width 1.5) (layer B.Cu) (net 4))
 (segment (start 118.03 60.96) (end 118.03 50.88) (width 1.5) (layer B.Cu) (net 4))
 (segment (start 77.55 50.88) (end 77.47 50.96) (width 1.5) (layer B.Cu) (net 4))
 (segment (start 77.47 50.96) (end 77.47 76.2) (width 1.5) (layer B.Cu) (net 4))
 (segment (start 77.47 76.2) (end 77.55 76.28) (width 1.5) (layer B.Cu) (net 4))
 (segment (start 77.55 76.28) (end 90.17 76.28) (width 1.5) (layer B.Cu) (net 4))
 (segment (start 118.03 50.88) (end 77.55 50.88) (width 1.5) (layer B.Cu) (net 4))
 (segment (start 77.55 93.9) (end 77.71 94.06) (width 1.5) (layer B.Cu) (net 4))
 (segment (start 77.71 94.06) (end 90.17 94.06) (width 1.5) (layer B.Cu) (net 4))
 (segment (start 77.55 76.28) (end 77.55 93.9) (width 1.5) (layer B.Cu) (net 4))
 (segment (start 77.55 93.98) (end 77.55 93.9) (width 1.5) (layer B.Cu) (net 4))
 (segment (start 77.55 113.11) (end 77.55 93.98) (width 1.5) (layer B.Cu) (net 4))
 (segment (start 90.17 113.11) (end 77.55 113.11) (width 1.5) (layer B.Cu) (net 4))
 (segment (start 77.47 139.7) (end 77.55 139.62) (width 1.5) (layer B.Cu) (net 4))
 (segment (start 77.55 139.62) (end 77.55 113.11) (width 1.5) (layer B.Cu) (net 4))
 (segment (start 153.67 139.7) (end 77.47 139.7) (width 1.5) (layer B.Cu) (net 4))
 (segment (start 185.166 83.566) (end 167.132 101.6) (width 1) (layer B.Cu) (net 5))
 (segment (start 167.132 101.6) (end 132.08 101.6) (width 1) (layer B.Cu) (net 5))
 (segment (start 132.08 101.6) (end 120.65 113.03) (width 1) (layer B.Cu) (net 5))
 (segment (start 120.65 114.3) (end 120.65 118.11) (width 1) (layer B.Cu) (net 5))
 (segment (start 120.65 113.03) (end 120.65 114.3) (width 1) (layer B.Cu) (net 5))
 (segment (start 185.166 71.12) (end 185.166 83.566) (width 1) (layer B.Cu) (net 5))
 (segment (start 107.95 114.3) (end 104.14 118.11) (width 1) (layer B.Cu) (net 5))
 (segment (start 104.14 118.11) (end 90.17 118.11) (width 1) (layer B.Cu) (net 5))
 (segment (start 120.65 114.3) (end 107.95 114.3) (width 1) (layer B.Cu) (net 5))
 (segment (start 182.626 81.534) (end 165.1 99.06) (width 1) (layer B.Cu) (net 6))
 (segment (start 165.1 99.06) (end 120.65 99.06) (width 1) (layer B.Cu) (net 6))
 (segment (start 182.626 71.12) (end 182.626 81.534) (width 1) (layer B.Cu) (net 6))
 (segment (start 120.65 95.25) (end 109.22 95.25) (width 1) (layer B.Cu) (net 6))
 (segment (start 109.22 95.25) (end 105.41 99.06) (width 1) (layer B.Cu) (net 6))
 (segment (start 105.41 99.06) (end 90.17 99.06) (width 1) (layer B.Cu) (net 6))
 (segment (start 120.65 99.06) (end 120.65 95.25) (width 1) (layer B.Cu) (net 6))
 (segment (start 100.33 81.28) (end 90.17 81.28) (width 1) (layer B.Cu) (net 7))
 (segment (start 100.33 85.09) (end 100.33 81.28) (width 1) (layer B.Cu) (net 7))
 (segment (start 102.87 87.63) (end 100.33 85.09) (width 1) (layer B.Cu) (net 7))
 (segment (start 120.65 87.63) (end 102.87 87.63) (width 1) (layer B.Cu) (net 7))
 (segment (start 120.65 90.17) (end 120.65 87.63) (width 1) (layer B.Cu) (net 7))
 (segment (start 180.086 80.264) (end 170.18 90.17) (width 1) (layer B.Cu) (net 7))
 (segment (start 170.18 90.17) (end 120.65 90.17) (width 1) (layer B.Cu) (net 7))
 (segment (start 180.086 71.12) (end 180.086 80.264) (width 1) (layer B.Cu) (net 7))
 (segment (start 213.36 66.04) (end 213.36 59.69) (width 1) (layer B.Cu) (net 8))
 (segment (start 212.09 67.31) (end 213.36 66.04) (width 1) (layer B.Cu) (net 8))
 (segment (start 205.74 67.31) (end 212.09 67.31) (width 1) (layer B.Cu) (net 8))
 (segment (start 204.47 71.12) (end 204.47 68.58) (width 1) (layer B.Cu) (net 8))
 (segment (start 204.47 68.58) (end 205.74 67.31) (width 1) (layer B.Cu) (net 8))
 (segment (start 207.01 71.12) (end 214.63 71.12) (width 1) (layer B.Cu) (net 9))
 (segment (start 215.9 69.85) (end 215.9 59.69) (width 1) (layer B.Cu) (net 9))
 (segment (start 214.63 71.12) (end 215.9 69.85) (width 1) (layer B.Cu) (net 9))
 (segment (start 152.4 118.11) (end 151.13 119.38) (width 1) (layer B.Cu) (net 10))
 (segment (start 156.21 115.57) (end 152.4 118.11) (width 1) (layer B.Cu) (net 10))
 (segment (start 184.15 115.57) (end 156.21 115.57) (width 1) (layer B.Cu) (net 10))
 (via (at 184.15 115.57) (size 2) (layers F.Cu B.Cu) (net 10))
 (segment (start 189.23 115.57) (end 184.15 115.57) (width 1) (layer F.Cu) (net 10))
 (via (at 189.23 115.57) (size 2) (layers F.Cu B.Cu) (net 10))
 (segment (start 193.04 115.57) (end 189.23 115.57) (width 1) (layer B.Cu) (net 10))
 (segment (start 194.31 115.57) (end 193.04 115.57) (width 1) (layer B.Cu) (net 10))
 (segment (start 194.31 119.38) (end 194.31 115.57) (width 1) (layer B.Cu) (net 10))
 (segment (start 151.13 119.38) (end 151.13 129.54) (width 1) (layer B.Cu) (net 10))
 (segment (start 140.97 80.01) (end 168.91 80.01) (width 1) (layer B.Cu) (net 20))
 (segment (start 172.72 76.2) (end 172.72 71.374) (width 1) (layer B.Cu) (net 20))
 (segment (start 168.91 80.01) (end 172.72 76.2) (width 1) (layer B.Cu) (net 20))
 (segment (start 172.72 71.374) (end 172.466 71.12) (width 1) (layer B.Cu) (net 20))
 (segment (start 196.85 71.12) (end 196.85 66.04) (width 1) (layer B.Cu) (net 11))
 (segment (start 189.15 62.15) (end 189.15 59.69) (width 1) (layer B.Cu) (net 11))
 (segment (start 193.04 66.04) (end 189.15 62.15) (width 1) (layer B.Cu) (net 11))
 (segment (start 196.85 66.04) (end 193.04 66.04) (width 1) (layer B.Cu) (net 11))
 (segment (start 201.93 71.12) (end 201.93 66.04) (width 1) (layer B.Cu) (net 12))
 (segment (start 194.15 63.34) (end 194.15 59.69) (width 1) (layer B.Cu) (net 12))
 (segment (start 194.31 63.5) (end 194.15 63.34) (width 1) (layer B.Cu) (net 12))
 (segment (start 199.39 63.5) (end 194.31 63.5) (width 1) (layer B.Cu) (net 12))
 (segment (start 201.93 66.04) (end 199.39 63.5) (width 1) (layer B.Cu) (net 12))
 (segment (start 186.69 68.58) (end 171.45 68.58) (width 1) (layer B.Cu) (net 13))
 (segment (start 171.45 68.58) (end 168.91 66.04) (width 1) (layer B.Cu) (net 13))
 (segment (start 168.91 66.04) (end 158.75 66.04) (width 1) (layer B.Cu) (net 13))
 (segment (start 158.75 66.04) (end 154.94 62.23) (width 1) (layer B.Cu) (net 13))
 (segment (start 154.94 62.23) (end 154.94 59.69) (width 1) (layer B.Cu) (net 13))
 (segment (start 189.23 71.12) (end 186.69 68.58) (width 1) (layer B.Cu) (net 13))
 (segment (start 163.83 63.5) (end 160.02 59.69) (width 1) (layer B.Cu) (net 14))
 (segment (start 170.18 63.5) (end 163.83 63.5) (width 1) (layer B.Cu) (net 14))
 (segment (start 172.72 66.04) (end 170.18 63.5) (width 1) (layer B.Cu) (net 14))
 (segment (start 187.96 66.04) (end 172.72 66.04) (width 1) (layer B.Cu) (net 14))
 (segment (start 191.77 69.85) (end 187.96 66.04) (width 1) (layer B.Cu) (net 14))
 (segment (start 191.77 71.12) (end 191.77 69.85) (width 1) (layer B.Cu) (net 14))
 (segment (start 173.99 129.46) (end 174.07 129.54) (width 1) (layer B.Cu) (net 16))
 (segment (start 196.85 123.19) (end 185.42 123.19) (width 1) (layer B.Cu) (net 16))
 (segment (start 185.42 123.19) (end 182.88 125.73) (width 1) (layer B.Cu) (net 16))
 (segment (start 182.88 125.73) (end 175.26 125.73) (width 1) (layer B.Cu) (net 16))
 (segment (start 175.26 125.73) (end 173.99 127) (width 1) (layer B.Cu) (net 16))
 (segment (start 173.99 127) (end 173.99 129.46) (width 1) (layer B.Cu) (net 16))
 (segment (start 196.85 119.38) (end 196.85 123.19) (width 1) (layer B.Cu) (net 16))
 (segment (start 200.74 128.35) (end 200.74 129.54) (width 1) (layer B.Cu) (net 17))
 (segment (start 199.39 127) (end 200.74 128.35) (width 1) (layer B.Cu) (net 17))
 (segment (start 199.39 119.38) (end 199.39 127) (width 1) (layer B.Cu) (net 17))
 (segment (start 177.546 78.486) (end 170.942 85.09) (width 1) (layer B.Cu) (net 19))
 (segment (start 170.942 85.09) (end 104.14 85.09) (width 1) (layer B.Cu) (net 19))
 (segment (start 104.14 85.09) (end 102.87 83.82) (width 1) (layer B.Cu) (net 19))
 (segment (start 102.87 83.82) (end 102.87 66.04) (width 1) (layer B.Cu) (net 19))
 (segment (start 102.87 66.04) (end 101.6 64.77) (width 1) (layer B.Cu) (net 19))
 (segment (start 101.6 64.77) (end 90.17 64.77) (width 1) (layer B.Cu) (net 19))
 (segment (start 177.546 71.12) (end 177.546 78.486) (width 1) (layer B.Cu) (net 19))
 (segment (start 199.39 81.28) (end 173.99 106.68) (width 1) (layer B.Cu) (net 18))
 (segment (start 173.99 106.68) (end 146.05 106.68) (width 1) (layer B.Cu) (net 18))
 (segment (start 146.05 106.68) (end 132.08 120.65) (width 1) (layer B.Cu) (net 18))
 (segment (start 132.08 120.65) (end 132.08 129.54) (width 1) (layer B.Cu) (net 18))
 (segment (start 199.39 71.12) (end 199.39 81.28) (width 1) (layer B.Cu) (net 18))
 (segment (start 194.31 71.12) (end 194.31 68.58) (width 1) (layer B.Cu) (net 15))
 (segment (start 173.99 63.5) (end 170.18 59.69) (width 1) (layer B.Cu) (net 15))
 (segment (start 187.96 63.5) (end 173.99 63.5) (width 1) (layer B.Cu) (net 15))
 (segment (start 193.04 68.58) (end 187.96 63.5) (width 1) (layer B.Cu) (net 15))
 (segment (start 194.31 68.58) (end 193.04 68.58) (width 1) (layer B.Cu) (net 15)))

